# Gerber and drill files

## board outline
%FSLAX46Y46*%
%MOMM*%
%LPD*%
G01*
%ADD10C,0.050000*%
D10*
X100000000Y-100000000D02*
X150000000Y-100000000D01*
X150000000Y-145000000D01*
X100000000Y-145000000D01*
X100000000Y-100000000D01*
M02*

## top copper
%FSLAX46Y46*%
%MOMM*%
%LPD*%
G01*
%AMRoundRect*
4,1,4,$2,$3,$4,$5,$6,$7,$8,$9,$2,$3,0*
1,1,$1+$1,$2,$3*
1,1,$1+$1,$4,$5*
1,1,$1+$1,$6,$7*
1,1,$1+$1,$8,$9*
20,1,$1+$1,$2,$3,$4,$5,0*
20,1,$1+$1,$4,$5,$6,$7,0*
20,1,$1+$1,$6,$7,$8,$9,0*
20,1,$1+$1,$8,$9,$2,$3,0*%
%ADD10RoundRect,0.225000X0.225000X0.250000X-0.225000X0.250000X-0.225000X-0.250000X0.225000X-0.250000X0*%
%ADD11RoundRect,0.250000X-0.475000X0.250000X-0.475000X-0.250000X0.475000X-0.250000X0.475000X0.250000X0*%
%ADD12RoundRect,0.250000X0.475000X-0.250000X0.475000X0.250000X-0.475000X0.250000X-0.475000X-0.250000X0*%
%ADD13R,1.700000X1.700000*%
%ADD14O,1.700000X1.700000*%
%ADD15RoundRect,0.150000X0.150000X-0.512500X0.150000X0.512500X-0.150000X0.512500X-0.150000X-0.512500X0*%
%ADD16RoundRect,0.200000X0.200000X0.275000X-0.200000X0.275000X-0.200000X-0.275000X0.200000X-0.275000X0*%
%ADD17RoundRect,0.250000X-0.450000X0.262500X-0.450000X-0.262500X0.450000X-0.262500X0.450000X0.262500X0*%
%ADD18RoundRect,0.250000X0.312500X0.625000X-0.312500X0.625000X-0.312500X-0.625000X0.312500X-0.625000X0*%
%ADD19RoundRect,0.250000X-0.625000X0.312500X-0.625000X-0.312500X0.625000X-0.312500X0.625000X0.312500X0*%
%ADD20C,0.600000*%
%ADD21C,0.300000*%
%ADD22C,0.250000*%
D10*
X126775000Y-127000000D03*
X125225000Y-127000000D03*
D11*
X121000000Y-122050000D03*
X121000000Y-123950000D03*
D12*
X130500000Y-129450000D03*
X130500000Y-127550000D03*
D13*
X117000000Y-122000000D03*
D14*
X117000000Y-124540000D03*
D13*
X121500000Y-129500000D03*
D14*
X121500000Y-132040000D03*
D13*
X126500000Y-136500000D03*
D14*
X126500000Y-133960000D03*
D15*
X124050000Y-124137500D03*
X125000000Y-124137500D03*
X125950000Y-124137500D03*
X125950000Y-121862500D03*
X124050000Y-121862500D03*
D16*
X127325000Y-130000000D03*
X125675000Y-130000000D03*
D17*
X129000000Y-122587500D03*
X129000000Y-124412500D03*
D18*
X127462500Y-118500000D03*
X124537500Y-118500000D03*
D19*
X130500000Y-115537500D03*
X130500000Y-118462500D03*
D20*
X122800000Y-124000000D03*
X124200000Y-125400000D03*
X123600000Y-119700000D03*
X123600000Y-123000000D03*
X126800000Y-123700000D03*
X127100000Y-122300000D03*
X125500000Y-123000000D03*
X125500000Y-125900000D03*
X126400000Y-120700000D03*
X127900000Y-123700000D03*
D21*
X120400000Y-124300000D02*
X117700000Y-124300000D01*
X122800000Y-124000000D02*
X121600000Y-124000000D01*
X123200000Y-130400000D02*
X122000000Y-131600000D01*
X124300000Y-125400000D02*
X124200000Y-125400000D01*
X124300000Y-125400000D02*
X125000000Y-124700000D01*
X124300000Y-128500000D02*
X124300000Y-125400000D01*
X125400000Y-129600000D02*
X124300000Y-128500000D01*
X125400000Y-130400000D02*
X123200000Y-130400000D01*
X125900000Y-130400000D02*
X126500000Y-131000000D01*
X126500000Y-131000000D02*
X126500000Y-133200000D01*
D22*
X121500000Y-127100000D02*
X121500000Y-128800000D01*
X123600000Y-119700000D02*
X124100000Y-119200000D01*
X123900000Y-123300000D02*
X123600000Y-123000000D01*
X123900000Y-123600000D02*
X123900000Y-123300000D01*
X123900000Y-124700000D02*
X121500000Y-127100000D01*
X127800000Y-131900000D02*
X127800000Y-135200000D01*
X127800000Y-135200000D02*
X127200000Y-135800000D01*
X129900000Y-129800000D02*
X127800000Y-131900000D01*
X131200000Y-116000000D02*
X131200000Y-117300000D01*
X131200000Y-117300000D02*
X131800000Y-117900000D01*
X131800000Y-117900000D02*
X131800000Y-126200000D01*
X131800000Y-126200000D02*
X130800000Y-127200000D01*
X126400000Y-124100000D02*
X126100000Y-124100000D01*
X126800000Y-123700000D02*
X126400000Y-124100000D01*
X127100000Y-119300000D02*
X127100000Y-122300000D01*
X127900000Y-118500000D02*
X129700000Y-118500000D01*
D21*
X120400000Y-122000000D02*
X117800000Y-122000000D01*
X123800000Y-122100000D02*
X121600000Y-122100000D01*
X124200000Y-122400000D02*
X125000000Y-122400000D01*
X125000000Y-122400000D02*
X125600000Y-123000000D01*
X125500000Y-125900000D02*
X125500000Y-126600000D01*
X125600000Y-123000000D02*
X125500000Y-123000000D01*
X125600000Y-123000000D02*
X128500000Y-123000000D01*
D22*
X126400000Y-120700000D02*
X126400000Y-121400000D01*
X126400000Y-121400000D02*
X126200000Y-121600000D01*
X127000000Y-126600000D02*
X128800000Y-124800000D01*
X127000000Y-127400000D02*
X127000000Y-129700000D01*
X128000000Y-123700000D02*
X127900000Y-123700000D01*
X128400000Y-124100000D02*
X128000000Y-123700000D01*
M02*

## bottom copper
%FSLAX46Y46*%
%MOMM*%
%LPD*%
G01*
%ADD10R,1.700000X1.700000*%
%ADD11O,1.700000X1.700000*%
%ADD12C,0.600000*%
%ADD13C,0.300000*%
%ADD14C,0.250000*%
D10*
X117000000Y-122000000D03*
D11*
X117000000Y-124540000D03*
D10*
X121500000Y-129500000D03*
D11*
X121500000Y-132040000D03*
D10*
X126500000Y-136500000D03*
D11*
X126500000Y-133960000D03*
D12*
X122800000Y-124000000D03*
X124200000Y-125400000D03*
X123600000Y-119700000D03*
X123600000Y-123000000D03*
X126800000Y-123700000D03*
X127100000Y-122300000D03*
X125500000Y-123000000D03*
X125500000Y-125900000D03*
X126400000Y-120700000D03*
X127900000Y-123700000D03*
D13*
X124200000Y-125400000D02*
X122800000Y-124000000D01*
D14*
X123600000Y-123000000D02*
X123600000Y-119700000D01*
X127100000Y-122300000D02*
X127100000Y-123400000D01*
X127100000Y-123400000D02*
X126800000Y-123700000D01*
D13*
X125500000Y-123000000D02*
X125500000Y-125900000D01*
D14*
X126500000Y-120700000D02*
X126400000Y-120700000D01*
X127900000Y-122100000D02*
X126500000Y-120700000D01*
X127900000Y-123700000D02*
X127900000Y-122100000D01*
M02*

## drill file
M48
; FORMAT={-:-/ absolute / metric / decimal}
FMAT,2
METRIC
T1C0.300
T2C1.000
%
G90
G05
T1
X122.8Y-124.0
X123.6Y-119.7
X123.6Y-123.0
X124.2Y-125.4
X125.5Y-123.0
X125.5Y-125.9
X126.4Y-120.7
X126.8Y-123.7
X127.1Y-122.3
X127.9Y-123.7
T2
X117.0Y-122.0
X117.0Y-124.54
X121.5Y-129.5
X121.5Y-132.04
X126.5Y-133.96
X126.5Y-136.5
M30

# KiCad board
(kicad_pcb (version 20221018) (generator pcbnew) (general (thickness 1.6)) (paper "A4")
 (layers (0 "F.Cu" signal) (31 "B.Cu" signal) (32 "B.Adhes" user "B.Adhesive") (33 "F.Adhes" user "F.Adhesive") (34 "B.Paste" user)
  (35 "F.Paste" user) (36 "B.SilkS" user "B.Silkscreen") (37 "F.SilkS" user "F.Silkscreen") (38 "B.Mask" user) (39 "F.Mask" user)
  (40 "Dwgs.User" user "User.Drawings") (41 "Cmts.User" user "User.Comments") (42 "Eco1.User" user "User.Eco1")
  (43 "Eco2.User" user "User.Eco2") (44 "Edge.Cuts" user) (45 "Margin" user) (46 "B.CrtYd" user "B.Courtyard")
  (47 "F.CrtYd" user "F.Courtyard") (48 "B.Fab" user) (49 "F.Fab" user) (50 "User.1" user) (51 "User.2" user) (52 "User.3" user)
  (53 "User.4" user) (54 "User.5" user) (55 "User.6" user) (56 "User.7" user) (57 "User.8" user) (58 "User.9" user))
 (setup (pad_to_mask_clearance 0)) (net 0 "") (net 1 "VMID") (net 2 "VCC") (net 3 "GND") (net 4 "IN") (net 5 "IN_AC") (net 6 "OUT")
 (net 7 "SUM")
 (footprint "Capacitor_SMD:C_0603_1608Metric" (layer "F.Cu") (at 126 127 180)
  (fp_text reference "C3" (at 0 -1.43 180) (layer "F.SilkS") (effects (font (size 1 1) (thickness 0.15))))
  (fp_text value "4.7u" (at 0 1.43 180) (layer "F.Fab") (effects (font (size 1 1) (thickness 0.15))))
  (pad "1" smd roundrect (at -0.775 0 180) (size 0.9 0.95) (layers "F.Cu" "F.Paste" "F.Mask") (roundrect_rratio 0.25) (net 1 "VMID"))
  (pad "2" smd roundrect (at 0.775 0 180) (size 0.9 0.95) (layers "F.Cu" "F.Paste" "F.Mask") (roundrect_rratio 0.25) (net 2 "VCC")))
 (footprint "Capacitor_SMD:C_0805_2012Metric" (layer "F.Cu") (at 121 123 -90)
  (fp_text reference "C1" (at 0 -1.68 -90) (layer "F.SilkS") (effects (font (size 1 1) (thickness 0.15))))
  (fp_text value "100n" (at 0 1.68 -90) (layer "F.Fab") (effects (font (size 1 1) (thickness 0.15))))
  (pad "1" smd roundrect (at -0.95 0 270) (size 1 1.45) (layers "F.Cu" "F.Paste" "F.Mask") (roundrect_rratio 0.25) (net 2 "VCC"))
  (pad "2" smd roundrect (at 0.95 0 270) (size 1 1.45) (layers "F.Cu" "F.Paste" "F.Mask") (roundrect_rratio 0.25) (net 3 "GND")))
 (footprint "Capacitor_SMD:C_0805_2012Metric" (layer "F.Cu") (at 130.5 128.5 90)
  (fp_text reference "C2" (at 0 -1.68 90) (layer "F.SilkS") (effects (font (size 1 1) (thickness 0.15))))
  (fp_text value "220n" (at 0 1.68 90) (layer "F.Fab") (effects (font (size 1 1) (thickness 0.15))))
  (pad "1" smd roundrect (at -0.95 0 90) (size 1 1.45) (layers "F.Cu" "F.Paste" "F.Mask") (roundrect_rratio 0.25) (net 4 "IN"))
  (pad "2" smd roundrect (at 0.95 0 90) (size 1 1.45) (layers "F.Cu" "F.Paste" "F.Mask") (roundrect_rratio 0.25) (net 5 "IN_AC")))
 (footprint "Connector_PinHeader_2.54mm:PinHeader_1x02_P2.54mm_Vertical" (layer "F.Cu") (at 117 122)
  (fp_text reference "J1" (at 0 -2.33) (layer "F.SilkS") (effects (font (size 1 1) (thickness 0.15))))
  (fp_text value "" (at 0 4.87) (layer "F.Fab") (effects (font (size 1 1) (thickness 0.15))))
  (pad "1" thru_hole rect (at 0 0) (size 1.7 1.7) (drill 1) (layers "*.Cu" "*.Mask") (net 2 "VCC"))
  (pad "2" thru_hole oval (at 0 2.54) (size 1.7 1.7) (drill 1) (layers "*.Cu" "*.Mask") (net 3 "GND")))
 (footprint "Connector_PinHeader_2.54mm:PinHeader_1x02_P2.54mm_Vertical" (layer "F.Cu") (at 121.5 129.5)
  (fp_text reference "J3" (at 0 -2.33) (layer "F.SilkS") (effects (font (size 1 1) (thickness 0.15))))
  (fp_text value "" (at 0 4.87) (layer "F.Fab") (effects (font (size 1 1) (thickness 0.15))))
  (pad "1" thru_hole rect (at 0 0) (size 1.7 1.7) (drill 1) (layers "*.Cu" "*.Mask") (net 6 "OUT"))
  (pad "2" thru_hole oval (at 0 2.54) (size 1.7 1.7) (drill 1) (layers "*.Cu" "*.Mask") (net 3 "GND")))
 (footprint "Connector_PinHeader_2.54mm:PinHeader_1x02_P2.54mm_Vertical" (layer "F.Cu") (at 126.5 136.5 180)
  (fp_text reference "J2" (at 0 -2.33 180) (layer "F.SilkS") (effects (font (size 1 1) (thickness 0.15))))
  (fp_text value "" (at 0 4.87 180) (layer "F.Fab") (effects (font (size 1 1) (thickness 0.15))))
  (pad "1" thru_hole rect (at 0 0 180) (size 1.7 1.7) (drill 1) (layers "*.Cu" "*.Mask") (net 4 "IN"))
  (pad "2" thru_hole oval (at 0 2.54 180) (size 1.7 1.7) (drill 1) (layers "*.Cu" "*.Mask") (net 3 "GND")))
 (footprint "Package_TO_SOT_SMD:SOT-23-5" (layer "F.Cu") (at 125 123 90)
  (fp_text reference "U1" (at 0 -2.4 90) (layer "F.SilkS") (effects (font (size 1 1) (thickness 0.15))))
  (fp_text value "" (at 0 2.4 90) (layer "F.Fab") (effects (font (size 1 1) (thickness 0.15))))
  (pad "1" smd roundrect (at -1.1375 -0.95 90) (size 1.325 0.6) (layers "F.Cu" "F.Paste" "F.Mask") (roundrect_rratio 0.25) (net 6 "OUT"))
  (pad "2" smd roundrect (at -1.1375 0 90) (size 1.325 0.6) (layers "F.Cu" "F.Paste" "F.Mask") (roundrect_rratio 0.25) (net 3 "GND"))
  (pad "3" smd roundrect (at -1.1375 0.95 90) (size 1.325 0.6) (layers "F.Cu" "F.Paste" "F.Mask") (roundrect_rratio 0.25) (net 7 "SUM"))
  (pad "4" smd roundrect (at 1.1375 0.95 90) (size 1.325 0.6) (layers "F.Cu" "F.Paste" "F.Mask") (roundrect_rratio 0.25) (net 1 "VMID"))
  (pad "5" smd roundrect (at 1.1375 -0.95 90) (size 1.325 0.6) (layers "F.Cu" "F.Paste" "F.Mask") (roundrect_rratio 0.25) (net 2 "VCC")))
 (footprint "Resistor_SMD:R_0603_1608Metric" (layer "F.Cu") (at 126.5 130 180)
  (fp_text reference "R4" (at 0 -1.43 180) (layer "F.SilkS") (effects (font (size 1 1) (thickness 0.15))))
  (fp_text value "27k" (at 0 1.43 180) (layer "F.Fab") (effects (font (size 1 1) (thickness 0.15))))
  (pad "1" smd roundrect (at -0.825 0 180) (size 0.8 0.95) (layers "F.Cu" "F.Paste" "F.Mask") (roundrect_rratio 0.25) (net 1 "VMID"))
  (pad "2" smd roundrect (at 0.825 0 180) (size 0.8 0.95) (layers "F.Cu" "F.Paste" "F.Mask") (roundrect_rratio 0.25) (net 3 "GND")))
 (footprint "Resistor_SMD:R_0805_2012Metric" (layer "F.Cu") (at 129 123.5 -90)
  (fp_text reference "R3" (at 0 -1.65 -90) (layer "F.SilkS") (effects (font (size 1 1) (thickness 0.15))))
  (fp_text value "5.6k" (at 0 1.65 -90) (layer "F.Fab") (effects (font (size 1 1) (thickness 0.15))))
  (pad "1" smd roundrect (at -0.9125 0 270) (size 1.025 1.4) (layers "F.Cu" "F.Paste" "F.Mask") (roundrect_rratio 0.243902) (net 2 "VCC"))
  (pad "2" smd roundrect (at 0.9125 0 270) (size 1.025 1.4) (layers "F.Cu" "F.Paste" "F.Mask") (roundrect_rratio 0.243902) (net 1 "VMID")))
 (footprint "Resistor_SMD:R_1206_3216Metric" (layer "F.Cu") (at 126 118.5 180)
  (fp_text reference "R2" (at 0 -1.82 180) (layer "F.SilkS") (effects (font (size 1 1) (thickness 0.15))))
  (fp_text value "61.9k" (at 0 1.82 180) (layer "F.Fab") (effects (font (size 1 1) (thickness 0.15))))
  (pad "1" smd roundrect (at -1.4625 0 180) (size 1.125 1.75) (layers "F.Cu" "F.Paste" "F.Mask") (roundrect_rratio 0.222222) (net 7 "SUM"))
  (pad "2" smd roundrect (at 1.4625 0 180) (size 1.125 1.75) (layers "F.Cu" "F.Paste" "F.Mask") (roundrect_rratio 0.222222) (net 6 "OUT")))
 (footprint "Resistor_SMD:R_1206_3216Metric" (layer "F.Cu") (at 130.5 117 -90)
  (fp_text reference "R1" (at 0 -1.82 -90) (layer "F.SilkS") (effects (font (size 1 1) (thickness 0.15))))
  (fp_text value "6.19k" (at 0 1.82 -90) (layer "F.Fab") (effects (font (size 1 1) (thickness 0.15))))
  (pad "1" smd roundrect (at -1.4625 0 270) (size 1.125 1.75) (layers "F.Cu" "F.Paste" "F.Mask") (roundrect_rratio 0.222222) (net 5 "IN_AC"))
  (pad "2" smd roundrect (at 1.4625 0 270) (size 1.125 1.75) (layers "F.Cu" "F.Paste" "F.Mask") (roundrect_rratio 0.222222) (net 7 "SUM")))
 (gr_rect (start 100 100) (end 150 145) (stroke (width 0.05) (type default)) (fill none) (layer "Edge.Cuts"))
 (segment (start 120.4 124.3) (end 117.7 124.3) (width 0.3) (layer "F.Cu") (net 3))
 (segment (start 122.8 124) (end 121.6 124) (width 0.3) (layer "F.Cu") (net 3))
 (segment (start 123.2 130.4) (end 122 131.6) (width 0.3) (layer "F.Cu") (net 3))
 (segment (start 124.3 125.4) (end 124.2 125.4) (width 0.3) (layer "F.Cu") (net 3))
 (segment (start 124.3 125.4) (end 125 124.7) (width 0.3) (layer "F.Cu") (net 3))
 (segment (start 124.3 128.5) (end 124.3 125.4) (width 0.3) (layer "F.Cu") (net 3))
 (segment (start 125.4 129.6) (end 124.3 128.5) (width 0.3) (layer "F.Cu") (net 3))
 (segment (start 125.4 130.4) (end 123.2 130.4) (width 0.3) (layer "F.Cu") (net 3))
 (segment (start 125.9 130.4) (end 126.5 131) (width 0.3) (layer "F.Cu") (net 3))
 (segment (start 126.5 131) (end 126.5 133.2) (width 0.3) (layer "F.Cu") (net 3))
 (via (at 122.8 124) (size 0.6) (drill 0.3) (layers "F.Cu" "B.Cu") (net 3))
 (via (at 124.2 125.4) (size 0.6) (drill 0.3) (layers "F.Cu" "B.Cu") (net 3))
 (segment (start 121.5 127.1) (end 121.5 128.8) (width 0.25) (layer "F.Cu") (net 6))
 (segment (start 123.6 119.7) (end 124.1 119.2) (width 0.25) (layer "F.Cu") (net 6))
 (segment (start 123.9 123.3) (end 123.6 123) (width 0.25) (layer "F.Cu") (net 6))
 (segment (start 123.9 123.6) (end 123.9 123.3) (width 0.25) (layer "F.Cu") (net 6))
 (segment (start 123.9 124.7) (end 121.5 127.1) (width 0.25) (layer "F.Cu") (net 6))
 (segment (start 124.2 125.4) (end 122.8 124) (width 0.3) (layer "B.Cu") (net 3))
 (segment (start 127.8 131.9) (end 127.8 135.2) (width 0.25) (layer "F.Cu") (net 4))
 (segment (start 127.8 135.2) (end 127.2 135.8) (width 0.25) (layer "F.Cu") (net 4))
 (segment (start 129.9 129.8) (end 127.8 131.9) (width 0.25) (layer "F.Cu") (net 4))
 (segment (start 131.2 116) (end 131.2 117.3) (width 0.25) (layer "F.Cu") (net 5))
 (segment (start 131.2 117.3) (end 131.8 117.9) (width 0.25) (layer "F.Cu") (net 5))
 (segment (start 131.8 117.9) (end 131.8 126.2) (width 0.25) (layer "F.Cu") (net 5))
 (segment (start 131.8 126.2) (end 130.8 127.2) (width 0.25) (layer "F.Cu") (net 5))
 (via (at 123.6 119.7) (size 0.6) (drill 0.3) (layers "F.Cu" "B.Cu") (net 6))
 (via (at 123.6 123) (size 0.6) (drill 0.3) (layers "F.Cu" "B.Cu") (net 6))
 (segment (start 123.6 123) (end 123.6 119.7) (width 0.25) (layer "B.Cu") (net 6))
 (segment (start 126.4 124.1) (end 126.1 124.1) (width 0.25) (layer "F.Cu") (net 7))
 (segment (start 126.8 123.7) (end 126.4 124.1) (width 0.25) (layer "F.Cu") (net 7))
 (segment (start 127.1 119.3) (end 127.1 122.3) (width 0.25) (layer "F.Cu") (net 7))
 (segment (start 127.9 118.5) (end 129.7 118.5) (width 0.25) (layer "F.Cu") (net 7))
 (via (at 126.8 123.7) (size 0.6) (drill 0.3) (layers "F.Cu" "B.Cu") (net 7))
 (via (at 127.1 122.3) (size 0.6) (drill 0.3) (layers "F.Cu" "B.Cu") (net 7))
 (segment (start 120.4 122) (end 117.8 122) (width 0.3) (layer "F.Cu") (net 2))
 (segment (start 123.8 122.1) (end 121.6 122.1) (width 0.3) (layer "F.Cu") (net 2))
 (segment (start 124.2 122.4) (end 125 122.4) (width 0.3) (layer "F.Cu") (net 2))
 (segment (start 125 122.4) (end 125.6 123) (width 0.3) (layer "F.Cu") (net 2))
 (segment (start 125.5 125.9) (end 125.5 126.6) (width 0.3) (layer "F.Cu") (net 2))
 (segment (start 125.6 123) (end 125.5 123) (width 0.3) (layer "F.Cu") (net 2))
 (segment (start 125.6 123) (end 128.5 123) (width 0.3) (layer "F.Cu") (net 2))
 (segment (start 127.1 122.3) (end 127.1 123.4) (width 0.25) (layer "B.Cu") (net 7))
 (segment (start 127.1 123.4) (end 126.8 123.7) (width 0.25) (layer "B.Cu") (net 7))
 (via (at 125.5 123) (size 0.6) (drill 0.3) (layers "F.Cu" "B.Cu") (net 2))
 (via (at 125.5 125.9) (size 0.6) (drill 0.3) (layers "F.Cu" "B.Cu") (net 2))
 (segment (start 125.5 123) (end 125.5 125.9) (width 0.3) (layer "B.Cu") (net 2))
 (segment (start 126.4 120.7) (end 126.4 121.4) (width 0.25) (layer "F.Cu") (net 1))
 (segment (start 126.4 121.4) (end 126.2 121.6) (width 0.25) (layer "F.Cu") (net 1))
 (segment (start 127 126.6) (end 128.8 124.8) (width 0.25) (layer "F.Cu") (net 1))
 (segment (start 127 127.4) (end 127 129.7) (width 0.25) (layer "F.Cu") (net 1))
 (segment (start 128 123.7) (end 127.9 123.7) (width 0.25) (layer "F.Cu") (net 1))
 (segment (start 128.4 124.1) (end 128 123.7) (width 0.25) (layer "F.Cu") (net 1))
 (via (at 126.4 120.7) (size 0.6) (drill 0.3) (layers "F.Cu" "B.Cu") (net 1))
 (via (at 127.9 123.7) (size 0.6) (drill 0.3) (layers "F.Cu" "B.Cu") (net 1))
 (segment (start 126.5 120.7) (end 126.4 120.7) (width 0.25) (layer "B.Cu") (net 1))
 (segment (start 127.9 122.1) (end 126.5 120.7) (width 0.25) (layer "B.Cu") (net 1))
 (segment (start 127.9 123.7) (end 127.9 122.1) (width 0.25) (layer "B.Cu") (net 1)))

